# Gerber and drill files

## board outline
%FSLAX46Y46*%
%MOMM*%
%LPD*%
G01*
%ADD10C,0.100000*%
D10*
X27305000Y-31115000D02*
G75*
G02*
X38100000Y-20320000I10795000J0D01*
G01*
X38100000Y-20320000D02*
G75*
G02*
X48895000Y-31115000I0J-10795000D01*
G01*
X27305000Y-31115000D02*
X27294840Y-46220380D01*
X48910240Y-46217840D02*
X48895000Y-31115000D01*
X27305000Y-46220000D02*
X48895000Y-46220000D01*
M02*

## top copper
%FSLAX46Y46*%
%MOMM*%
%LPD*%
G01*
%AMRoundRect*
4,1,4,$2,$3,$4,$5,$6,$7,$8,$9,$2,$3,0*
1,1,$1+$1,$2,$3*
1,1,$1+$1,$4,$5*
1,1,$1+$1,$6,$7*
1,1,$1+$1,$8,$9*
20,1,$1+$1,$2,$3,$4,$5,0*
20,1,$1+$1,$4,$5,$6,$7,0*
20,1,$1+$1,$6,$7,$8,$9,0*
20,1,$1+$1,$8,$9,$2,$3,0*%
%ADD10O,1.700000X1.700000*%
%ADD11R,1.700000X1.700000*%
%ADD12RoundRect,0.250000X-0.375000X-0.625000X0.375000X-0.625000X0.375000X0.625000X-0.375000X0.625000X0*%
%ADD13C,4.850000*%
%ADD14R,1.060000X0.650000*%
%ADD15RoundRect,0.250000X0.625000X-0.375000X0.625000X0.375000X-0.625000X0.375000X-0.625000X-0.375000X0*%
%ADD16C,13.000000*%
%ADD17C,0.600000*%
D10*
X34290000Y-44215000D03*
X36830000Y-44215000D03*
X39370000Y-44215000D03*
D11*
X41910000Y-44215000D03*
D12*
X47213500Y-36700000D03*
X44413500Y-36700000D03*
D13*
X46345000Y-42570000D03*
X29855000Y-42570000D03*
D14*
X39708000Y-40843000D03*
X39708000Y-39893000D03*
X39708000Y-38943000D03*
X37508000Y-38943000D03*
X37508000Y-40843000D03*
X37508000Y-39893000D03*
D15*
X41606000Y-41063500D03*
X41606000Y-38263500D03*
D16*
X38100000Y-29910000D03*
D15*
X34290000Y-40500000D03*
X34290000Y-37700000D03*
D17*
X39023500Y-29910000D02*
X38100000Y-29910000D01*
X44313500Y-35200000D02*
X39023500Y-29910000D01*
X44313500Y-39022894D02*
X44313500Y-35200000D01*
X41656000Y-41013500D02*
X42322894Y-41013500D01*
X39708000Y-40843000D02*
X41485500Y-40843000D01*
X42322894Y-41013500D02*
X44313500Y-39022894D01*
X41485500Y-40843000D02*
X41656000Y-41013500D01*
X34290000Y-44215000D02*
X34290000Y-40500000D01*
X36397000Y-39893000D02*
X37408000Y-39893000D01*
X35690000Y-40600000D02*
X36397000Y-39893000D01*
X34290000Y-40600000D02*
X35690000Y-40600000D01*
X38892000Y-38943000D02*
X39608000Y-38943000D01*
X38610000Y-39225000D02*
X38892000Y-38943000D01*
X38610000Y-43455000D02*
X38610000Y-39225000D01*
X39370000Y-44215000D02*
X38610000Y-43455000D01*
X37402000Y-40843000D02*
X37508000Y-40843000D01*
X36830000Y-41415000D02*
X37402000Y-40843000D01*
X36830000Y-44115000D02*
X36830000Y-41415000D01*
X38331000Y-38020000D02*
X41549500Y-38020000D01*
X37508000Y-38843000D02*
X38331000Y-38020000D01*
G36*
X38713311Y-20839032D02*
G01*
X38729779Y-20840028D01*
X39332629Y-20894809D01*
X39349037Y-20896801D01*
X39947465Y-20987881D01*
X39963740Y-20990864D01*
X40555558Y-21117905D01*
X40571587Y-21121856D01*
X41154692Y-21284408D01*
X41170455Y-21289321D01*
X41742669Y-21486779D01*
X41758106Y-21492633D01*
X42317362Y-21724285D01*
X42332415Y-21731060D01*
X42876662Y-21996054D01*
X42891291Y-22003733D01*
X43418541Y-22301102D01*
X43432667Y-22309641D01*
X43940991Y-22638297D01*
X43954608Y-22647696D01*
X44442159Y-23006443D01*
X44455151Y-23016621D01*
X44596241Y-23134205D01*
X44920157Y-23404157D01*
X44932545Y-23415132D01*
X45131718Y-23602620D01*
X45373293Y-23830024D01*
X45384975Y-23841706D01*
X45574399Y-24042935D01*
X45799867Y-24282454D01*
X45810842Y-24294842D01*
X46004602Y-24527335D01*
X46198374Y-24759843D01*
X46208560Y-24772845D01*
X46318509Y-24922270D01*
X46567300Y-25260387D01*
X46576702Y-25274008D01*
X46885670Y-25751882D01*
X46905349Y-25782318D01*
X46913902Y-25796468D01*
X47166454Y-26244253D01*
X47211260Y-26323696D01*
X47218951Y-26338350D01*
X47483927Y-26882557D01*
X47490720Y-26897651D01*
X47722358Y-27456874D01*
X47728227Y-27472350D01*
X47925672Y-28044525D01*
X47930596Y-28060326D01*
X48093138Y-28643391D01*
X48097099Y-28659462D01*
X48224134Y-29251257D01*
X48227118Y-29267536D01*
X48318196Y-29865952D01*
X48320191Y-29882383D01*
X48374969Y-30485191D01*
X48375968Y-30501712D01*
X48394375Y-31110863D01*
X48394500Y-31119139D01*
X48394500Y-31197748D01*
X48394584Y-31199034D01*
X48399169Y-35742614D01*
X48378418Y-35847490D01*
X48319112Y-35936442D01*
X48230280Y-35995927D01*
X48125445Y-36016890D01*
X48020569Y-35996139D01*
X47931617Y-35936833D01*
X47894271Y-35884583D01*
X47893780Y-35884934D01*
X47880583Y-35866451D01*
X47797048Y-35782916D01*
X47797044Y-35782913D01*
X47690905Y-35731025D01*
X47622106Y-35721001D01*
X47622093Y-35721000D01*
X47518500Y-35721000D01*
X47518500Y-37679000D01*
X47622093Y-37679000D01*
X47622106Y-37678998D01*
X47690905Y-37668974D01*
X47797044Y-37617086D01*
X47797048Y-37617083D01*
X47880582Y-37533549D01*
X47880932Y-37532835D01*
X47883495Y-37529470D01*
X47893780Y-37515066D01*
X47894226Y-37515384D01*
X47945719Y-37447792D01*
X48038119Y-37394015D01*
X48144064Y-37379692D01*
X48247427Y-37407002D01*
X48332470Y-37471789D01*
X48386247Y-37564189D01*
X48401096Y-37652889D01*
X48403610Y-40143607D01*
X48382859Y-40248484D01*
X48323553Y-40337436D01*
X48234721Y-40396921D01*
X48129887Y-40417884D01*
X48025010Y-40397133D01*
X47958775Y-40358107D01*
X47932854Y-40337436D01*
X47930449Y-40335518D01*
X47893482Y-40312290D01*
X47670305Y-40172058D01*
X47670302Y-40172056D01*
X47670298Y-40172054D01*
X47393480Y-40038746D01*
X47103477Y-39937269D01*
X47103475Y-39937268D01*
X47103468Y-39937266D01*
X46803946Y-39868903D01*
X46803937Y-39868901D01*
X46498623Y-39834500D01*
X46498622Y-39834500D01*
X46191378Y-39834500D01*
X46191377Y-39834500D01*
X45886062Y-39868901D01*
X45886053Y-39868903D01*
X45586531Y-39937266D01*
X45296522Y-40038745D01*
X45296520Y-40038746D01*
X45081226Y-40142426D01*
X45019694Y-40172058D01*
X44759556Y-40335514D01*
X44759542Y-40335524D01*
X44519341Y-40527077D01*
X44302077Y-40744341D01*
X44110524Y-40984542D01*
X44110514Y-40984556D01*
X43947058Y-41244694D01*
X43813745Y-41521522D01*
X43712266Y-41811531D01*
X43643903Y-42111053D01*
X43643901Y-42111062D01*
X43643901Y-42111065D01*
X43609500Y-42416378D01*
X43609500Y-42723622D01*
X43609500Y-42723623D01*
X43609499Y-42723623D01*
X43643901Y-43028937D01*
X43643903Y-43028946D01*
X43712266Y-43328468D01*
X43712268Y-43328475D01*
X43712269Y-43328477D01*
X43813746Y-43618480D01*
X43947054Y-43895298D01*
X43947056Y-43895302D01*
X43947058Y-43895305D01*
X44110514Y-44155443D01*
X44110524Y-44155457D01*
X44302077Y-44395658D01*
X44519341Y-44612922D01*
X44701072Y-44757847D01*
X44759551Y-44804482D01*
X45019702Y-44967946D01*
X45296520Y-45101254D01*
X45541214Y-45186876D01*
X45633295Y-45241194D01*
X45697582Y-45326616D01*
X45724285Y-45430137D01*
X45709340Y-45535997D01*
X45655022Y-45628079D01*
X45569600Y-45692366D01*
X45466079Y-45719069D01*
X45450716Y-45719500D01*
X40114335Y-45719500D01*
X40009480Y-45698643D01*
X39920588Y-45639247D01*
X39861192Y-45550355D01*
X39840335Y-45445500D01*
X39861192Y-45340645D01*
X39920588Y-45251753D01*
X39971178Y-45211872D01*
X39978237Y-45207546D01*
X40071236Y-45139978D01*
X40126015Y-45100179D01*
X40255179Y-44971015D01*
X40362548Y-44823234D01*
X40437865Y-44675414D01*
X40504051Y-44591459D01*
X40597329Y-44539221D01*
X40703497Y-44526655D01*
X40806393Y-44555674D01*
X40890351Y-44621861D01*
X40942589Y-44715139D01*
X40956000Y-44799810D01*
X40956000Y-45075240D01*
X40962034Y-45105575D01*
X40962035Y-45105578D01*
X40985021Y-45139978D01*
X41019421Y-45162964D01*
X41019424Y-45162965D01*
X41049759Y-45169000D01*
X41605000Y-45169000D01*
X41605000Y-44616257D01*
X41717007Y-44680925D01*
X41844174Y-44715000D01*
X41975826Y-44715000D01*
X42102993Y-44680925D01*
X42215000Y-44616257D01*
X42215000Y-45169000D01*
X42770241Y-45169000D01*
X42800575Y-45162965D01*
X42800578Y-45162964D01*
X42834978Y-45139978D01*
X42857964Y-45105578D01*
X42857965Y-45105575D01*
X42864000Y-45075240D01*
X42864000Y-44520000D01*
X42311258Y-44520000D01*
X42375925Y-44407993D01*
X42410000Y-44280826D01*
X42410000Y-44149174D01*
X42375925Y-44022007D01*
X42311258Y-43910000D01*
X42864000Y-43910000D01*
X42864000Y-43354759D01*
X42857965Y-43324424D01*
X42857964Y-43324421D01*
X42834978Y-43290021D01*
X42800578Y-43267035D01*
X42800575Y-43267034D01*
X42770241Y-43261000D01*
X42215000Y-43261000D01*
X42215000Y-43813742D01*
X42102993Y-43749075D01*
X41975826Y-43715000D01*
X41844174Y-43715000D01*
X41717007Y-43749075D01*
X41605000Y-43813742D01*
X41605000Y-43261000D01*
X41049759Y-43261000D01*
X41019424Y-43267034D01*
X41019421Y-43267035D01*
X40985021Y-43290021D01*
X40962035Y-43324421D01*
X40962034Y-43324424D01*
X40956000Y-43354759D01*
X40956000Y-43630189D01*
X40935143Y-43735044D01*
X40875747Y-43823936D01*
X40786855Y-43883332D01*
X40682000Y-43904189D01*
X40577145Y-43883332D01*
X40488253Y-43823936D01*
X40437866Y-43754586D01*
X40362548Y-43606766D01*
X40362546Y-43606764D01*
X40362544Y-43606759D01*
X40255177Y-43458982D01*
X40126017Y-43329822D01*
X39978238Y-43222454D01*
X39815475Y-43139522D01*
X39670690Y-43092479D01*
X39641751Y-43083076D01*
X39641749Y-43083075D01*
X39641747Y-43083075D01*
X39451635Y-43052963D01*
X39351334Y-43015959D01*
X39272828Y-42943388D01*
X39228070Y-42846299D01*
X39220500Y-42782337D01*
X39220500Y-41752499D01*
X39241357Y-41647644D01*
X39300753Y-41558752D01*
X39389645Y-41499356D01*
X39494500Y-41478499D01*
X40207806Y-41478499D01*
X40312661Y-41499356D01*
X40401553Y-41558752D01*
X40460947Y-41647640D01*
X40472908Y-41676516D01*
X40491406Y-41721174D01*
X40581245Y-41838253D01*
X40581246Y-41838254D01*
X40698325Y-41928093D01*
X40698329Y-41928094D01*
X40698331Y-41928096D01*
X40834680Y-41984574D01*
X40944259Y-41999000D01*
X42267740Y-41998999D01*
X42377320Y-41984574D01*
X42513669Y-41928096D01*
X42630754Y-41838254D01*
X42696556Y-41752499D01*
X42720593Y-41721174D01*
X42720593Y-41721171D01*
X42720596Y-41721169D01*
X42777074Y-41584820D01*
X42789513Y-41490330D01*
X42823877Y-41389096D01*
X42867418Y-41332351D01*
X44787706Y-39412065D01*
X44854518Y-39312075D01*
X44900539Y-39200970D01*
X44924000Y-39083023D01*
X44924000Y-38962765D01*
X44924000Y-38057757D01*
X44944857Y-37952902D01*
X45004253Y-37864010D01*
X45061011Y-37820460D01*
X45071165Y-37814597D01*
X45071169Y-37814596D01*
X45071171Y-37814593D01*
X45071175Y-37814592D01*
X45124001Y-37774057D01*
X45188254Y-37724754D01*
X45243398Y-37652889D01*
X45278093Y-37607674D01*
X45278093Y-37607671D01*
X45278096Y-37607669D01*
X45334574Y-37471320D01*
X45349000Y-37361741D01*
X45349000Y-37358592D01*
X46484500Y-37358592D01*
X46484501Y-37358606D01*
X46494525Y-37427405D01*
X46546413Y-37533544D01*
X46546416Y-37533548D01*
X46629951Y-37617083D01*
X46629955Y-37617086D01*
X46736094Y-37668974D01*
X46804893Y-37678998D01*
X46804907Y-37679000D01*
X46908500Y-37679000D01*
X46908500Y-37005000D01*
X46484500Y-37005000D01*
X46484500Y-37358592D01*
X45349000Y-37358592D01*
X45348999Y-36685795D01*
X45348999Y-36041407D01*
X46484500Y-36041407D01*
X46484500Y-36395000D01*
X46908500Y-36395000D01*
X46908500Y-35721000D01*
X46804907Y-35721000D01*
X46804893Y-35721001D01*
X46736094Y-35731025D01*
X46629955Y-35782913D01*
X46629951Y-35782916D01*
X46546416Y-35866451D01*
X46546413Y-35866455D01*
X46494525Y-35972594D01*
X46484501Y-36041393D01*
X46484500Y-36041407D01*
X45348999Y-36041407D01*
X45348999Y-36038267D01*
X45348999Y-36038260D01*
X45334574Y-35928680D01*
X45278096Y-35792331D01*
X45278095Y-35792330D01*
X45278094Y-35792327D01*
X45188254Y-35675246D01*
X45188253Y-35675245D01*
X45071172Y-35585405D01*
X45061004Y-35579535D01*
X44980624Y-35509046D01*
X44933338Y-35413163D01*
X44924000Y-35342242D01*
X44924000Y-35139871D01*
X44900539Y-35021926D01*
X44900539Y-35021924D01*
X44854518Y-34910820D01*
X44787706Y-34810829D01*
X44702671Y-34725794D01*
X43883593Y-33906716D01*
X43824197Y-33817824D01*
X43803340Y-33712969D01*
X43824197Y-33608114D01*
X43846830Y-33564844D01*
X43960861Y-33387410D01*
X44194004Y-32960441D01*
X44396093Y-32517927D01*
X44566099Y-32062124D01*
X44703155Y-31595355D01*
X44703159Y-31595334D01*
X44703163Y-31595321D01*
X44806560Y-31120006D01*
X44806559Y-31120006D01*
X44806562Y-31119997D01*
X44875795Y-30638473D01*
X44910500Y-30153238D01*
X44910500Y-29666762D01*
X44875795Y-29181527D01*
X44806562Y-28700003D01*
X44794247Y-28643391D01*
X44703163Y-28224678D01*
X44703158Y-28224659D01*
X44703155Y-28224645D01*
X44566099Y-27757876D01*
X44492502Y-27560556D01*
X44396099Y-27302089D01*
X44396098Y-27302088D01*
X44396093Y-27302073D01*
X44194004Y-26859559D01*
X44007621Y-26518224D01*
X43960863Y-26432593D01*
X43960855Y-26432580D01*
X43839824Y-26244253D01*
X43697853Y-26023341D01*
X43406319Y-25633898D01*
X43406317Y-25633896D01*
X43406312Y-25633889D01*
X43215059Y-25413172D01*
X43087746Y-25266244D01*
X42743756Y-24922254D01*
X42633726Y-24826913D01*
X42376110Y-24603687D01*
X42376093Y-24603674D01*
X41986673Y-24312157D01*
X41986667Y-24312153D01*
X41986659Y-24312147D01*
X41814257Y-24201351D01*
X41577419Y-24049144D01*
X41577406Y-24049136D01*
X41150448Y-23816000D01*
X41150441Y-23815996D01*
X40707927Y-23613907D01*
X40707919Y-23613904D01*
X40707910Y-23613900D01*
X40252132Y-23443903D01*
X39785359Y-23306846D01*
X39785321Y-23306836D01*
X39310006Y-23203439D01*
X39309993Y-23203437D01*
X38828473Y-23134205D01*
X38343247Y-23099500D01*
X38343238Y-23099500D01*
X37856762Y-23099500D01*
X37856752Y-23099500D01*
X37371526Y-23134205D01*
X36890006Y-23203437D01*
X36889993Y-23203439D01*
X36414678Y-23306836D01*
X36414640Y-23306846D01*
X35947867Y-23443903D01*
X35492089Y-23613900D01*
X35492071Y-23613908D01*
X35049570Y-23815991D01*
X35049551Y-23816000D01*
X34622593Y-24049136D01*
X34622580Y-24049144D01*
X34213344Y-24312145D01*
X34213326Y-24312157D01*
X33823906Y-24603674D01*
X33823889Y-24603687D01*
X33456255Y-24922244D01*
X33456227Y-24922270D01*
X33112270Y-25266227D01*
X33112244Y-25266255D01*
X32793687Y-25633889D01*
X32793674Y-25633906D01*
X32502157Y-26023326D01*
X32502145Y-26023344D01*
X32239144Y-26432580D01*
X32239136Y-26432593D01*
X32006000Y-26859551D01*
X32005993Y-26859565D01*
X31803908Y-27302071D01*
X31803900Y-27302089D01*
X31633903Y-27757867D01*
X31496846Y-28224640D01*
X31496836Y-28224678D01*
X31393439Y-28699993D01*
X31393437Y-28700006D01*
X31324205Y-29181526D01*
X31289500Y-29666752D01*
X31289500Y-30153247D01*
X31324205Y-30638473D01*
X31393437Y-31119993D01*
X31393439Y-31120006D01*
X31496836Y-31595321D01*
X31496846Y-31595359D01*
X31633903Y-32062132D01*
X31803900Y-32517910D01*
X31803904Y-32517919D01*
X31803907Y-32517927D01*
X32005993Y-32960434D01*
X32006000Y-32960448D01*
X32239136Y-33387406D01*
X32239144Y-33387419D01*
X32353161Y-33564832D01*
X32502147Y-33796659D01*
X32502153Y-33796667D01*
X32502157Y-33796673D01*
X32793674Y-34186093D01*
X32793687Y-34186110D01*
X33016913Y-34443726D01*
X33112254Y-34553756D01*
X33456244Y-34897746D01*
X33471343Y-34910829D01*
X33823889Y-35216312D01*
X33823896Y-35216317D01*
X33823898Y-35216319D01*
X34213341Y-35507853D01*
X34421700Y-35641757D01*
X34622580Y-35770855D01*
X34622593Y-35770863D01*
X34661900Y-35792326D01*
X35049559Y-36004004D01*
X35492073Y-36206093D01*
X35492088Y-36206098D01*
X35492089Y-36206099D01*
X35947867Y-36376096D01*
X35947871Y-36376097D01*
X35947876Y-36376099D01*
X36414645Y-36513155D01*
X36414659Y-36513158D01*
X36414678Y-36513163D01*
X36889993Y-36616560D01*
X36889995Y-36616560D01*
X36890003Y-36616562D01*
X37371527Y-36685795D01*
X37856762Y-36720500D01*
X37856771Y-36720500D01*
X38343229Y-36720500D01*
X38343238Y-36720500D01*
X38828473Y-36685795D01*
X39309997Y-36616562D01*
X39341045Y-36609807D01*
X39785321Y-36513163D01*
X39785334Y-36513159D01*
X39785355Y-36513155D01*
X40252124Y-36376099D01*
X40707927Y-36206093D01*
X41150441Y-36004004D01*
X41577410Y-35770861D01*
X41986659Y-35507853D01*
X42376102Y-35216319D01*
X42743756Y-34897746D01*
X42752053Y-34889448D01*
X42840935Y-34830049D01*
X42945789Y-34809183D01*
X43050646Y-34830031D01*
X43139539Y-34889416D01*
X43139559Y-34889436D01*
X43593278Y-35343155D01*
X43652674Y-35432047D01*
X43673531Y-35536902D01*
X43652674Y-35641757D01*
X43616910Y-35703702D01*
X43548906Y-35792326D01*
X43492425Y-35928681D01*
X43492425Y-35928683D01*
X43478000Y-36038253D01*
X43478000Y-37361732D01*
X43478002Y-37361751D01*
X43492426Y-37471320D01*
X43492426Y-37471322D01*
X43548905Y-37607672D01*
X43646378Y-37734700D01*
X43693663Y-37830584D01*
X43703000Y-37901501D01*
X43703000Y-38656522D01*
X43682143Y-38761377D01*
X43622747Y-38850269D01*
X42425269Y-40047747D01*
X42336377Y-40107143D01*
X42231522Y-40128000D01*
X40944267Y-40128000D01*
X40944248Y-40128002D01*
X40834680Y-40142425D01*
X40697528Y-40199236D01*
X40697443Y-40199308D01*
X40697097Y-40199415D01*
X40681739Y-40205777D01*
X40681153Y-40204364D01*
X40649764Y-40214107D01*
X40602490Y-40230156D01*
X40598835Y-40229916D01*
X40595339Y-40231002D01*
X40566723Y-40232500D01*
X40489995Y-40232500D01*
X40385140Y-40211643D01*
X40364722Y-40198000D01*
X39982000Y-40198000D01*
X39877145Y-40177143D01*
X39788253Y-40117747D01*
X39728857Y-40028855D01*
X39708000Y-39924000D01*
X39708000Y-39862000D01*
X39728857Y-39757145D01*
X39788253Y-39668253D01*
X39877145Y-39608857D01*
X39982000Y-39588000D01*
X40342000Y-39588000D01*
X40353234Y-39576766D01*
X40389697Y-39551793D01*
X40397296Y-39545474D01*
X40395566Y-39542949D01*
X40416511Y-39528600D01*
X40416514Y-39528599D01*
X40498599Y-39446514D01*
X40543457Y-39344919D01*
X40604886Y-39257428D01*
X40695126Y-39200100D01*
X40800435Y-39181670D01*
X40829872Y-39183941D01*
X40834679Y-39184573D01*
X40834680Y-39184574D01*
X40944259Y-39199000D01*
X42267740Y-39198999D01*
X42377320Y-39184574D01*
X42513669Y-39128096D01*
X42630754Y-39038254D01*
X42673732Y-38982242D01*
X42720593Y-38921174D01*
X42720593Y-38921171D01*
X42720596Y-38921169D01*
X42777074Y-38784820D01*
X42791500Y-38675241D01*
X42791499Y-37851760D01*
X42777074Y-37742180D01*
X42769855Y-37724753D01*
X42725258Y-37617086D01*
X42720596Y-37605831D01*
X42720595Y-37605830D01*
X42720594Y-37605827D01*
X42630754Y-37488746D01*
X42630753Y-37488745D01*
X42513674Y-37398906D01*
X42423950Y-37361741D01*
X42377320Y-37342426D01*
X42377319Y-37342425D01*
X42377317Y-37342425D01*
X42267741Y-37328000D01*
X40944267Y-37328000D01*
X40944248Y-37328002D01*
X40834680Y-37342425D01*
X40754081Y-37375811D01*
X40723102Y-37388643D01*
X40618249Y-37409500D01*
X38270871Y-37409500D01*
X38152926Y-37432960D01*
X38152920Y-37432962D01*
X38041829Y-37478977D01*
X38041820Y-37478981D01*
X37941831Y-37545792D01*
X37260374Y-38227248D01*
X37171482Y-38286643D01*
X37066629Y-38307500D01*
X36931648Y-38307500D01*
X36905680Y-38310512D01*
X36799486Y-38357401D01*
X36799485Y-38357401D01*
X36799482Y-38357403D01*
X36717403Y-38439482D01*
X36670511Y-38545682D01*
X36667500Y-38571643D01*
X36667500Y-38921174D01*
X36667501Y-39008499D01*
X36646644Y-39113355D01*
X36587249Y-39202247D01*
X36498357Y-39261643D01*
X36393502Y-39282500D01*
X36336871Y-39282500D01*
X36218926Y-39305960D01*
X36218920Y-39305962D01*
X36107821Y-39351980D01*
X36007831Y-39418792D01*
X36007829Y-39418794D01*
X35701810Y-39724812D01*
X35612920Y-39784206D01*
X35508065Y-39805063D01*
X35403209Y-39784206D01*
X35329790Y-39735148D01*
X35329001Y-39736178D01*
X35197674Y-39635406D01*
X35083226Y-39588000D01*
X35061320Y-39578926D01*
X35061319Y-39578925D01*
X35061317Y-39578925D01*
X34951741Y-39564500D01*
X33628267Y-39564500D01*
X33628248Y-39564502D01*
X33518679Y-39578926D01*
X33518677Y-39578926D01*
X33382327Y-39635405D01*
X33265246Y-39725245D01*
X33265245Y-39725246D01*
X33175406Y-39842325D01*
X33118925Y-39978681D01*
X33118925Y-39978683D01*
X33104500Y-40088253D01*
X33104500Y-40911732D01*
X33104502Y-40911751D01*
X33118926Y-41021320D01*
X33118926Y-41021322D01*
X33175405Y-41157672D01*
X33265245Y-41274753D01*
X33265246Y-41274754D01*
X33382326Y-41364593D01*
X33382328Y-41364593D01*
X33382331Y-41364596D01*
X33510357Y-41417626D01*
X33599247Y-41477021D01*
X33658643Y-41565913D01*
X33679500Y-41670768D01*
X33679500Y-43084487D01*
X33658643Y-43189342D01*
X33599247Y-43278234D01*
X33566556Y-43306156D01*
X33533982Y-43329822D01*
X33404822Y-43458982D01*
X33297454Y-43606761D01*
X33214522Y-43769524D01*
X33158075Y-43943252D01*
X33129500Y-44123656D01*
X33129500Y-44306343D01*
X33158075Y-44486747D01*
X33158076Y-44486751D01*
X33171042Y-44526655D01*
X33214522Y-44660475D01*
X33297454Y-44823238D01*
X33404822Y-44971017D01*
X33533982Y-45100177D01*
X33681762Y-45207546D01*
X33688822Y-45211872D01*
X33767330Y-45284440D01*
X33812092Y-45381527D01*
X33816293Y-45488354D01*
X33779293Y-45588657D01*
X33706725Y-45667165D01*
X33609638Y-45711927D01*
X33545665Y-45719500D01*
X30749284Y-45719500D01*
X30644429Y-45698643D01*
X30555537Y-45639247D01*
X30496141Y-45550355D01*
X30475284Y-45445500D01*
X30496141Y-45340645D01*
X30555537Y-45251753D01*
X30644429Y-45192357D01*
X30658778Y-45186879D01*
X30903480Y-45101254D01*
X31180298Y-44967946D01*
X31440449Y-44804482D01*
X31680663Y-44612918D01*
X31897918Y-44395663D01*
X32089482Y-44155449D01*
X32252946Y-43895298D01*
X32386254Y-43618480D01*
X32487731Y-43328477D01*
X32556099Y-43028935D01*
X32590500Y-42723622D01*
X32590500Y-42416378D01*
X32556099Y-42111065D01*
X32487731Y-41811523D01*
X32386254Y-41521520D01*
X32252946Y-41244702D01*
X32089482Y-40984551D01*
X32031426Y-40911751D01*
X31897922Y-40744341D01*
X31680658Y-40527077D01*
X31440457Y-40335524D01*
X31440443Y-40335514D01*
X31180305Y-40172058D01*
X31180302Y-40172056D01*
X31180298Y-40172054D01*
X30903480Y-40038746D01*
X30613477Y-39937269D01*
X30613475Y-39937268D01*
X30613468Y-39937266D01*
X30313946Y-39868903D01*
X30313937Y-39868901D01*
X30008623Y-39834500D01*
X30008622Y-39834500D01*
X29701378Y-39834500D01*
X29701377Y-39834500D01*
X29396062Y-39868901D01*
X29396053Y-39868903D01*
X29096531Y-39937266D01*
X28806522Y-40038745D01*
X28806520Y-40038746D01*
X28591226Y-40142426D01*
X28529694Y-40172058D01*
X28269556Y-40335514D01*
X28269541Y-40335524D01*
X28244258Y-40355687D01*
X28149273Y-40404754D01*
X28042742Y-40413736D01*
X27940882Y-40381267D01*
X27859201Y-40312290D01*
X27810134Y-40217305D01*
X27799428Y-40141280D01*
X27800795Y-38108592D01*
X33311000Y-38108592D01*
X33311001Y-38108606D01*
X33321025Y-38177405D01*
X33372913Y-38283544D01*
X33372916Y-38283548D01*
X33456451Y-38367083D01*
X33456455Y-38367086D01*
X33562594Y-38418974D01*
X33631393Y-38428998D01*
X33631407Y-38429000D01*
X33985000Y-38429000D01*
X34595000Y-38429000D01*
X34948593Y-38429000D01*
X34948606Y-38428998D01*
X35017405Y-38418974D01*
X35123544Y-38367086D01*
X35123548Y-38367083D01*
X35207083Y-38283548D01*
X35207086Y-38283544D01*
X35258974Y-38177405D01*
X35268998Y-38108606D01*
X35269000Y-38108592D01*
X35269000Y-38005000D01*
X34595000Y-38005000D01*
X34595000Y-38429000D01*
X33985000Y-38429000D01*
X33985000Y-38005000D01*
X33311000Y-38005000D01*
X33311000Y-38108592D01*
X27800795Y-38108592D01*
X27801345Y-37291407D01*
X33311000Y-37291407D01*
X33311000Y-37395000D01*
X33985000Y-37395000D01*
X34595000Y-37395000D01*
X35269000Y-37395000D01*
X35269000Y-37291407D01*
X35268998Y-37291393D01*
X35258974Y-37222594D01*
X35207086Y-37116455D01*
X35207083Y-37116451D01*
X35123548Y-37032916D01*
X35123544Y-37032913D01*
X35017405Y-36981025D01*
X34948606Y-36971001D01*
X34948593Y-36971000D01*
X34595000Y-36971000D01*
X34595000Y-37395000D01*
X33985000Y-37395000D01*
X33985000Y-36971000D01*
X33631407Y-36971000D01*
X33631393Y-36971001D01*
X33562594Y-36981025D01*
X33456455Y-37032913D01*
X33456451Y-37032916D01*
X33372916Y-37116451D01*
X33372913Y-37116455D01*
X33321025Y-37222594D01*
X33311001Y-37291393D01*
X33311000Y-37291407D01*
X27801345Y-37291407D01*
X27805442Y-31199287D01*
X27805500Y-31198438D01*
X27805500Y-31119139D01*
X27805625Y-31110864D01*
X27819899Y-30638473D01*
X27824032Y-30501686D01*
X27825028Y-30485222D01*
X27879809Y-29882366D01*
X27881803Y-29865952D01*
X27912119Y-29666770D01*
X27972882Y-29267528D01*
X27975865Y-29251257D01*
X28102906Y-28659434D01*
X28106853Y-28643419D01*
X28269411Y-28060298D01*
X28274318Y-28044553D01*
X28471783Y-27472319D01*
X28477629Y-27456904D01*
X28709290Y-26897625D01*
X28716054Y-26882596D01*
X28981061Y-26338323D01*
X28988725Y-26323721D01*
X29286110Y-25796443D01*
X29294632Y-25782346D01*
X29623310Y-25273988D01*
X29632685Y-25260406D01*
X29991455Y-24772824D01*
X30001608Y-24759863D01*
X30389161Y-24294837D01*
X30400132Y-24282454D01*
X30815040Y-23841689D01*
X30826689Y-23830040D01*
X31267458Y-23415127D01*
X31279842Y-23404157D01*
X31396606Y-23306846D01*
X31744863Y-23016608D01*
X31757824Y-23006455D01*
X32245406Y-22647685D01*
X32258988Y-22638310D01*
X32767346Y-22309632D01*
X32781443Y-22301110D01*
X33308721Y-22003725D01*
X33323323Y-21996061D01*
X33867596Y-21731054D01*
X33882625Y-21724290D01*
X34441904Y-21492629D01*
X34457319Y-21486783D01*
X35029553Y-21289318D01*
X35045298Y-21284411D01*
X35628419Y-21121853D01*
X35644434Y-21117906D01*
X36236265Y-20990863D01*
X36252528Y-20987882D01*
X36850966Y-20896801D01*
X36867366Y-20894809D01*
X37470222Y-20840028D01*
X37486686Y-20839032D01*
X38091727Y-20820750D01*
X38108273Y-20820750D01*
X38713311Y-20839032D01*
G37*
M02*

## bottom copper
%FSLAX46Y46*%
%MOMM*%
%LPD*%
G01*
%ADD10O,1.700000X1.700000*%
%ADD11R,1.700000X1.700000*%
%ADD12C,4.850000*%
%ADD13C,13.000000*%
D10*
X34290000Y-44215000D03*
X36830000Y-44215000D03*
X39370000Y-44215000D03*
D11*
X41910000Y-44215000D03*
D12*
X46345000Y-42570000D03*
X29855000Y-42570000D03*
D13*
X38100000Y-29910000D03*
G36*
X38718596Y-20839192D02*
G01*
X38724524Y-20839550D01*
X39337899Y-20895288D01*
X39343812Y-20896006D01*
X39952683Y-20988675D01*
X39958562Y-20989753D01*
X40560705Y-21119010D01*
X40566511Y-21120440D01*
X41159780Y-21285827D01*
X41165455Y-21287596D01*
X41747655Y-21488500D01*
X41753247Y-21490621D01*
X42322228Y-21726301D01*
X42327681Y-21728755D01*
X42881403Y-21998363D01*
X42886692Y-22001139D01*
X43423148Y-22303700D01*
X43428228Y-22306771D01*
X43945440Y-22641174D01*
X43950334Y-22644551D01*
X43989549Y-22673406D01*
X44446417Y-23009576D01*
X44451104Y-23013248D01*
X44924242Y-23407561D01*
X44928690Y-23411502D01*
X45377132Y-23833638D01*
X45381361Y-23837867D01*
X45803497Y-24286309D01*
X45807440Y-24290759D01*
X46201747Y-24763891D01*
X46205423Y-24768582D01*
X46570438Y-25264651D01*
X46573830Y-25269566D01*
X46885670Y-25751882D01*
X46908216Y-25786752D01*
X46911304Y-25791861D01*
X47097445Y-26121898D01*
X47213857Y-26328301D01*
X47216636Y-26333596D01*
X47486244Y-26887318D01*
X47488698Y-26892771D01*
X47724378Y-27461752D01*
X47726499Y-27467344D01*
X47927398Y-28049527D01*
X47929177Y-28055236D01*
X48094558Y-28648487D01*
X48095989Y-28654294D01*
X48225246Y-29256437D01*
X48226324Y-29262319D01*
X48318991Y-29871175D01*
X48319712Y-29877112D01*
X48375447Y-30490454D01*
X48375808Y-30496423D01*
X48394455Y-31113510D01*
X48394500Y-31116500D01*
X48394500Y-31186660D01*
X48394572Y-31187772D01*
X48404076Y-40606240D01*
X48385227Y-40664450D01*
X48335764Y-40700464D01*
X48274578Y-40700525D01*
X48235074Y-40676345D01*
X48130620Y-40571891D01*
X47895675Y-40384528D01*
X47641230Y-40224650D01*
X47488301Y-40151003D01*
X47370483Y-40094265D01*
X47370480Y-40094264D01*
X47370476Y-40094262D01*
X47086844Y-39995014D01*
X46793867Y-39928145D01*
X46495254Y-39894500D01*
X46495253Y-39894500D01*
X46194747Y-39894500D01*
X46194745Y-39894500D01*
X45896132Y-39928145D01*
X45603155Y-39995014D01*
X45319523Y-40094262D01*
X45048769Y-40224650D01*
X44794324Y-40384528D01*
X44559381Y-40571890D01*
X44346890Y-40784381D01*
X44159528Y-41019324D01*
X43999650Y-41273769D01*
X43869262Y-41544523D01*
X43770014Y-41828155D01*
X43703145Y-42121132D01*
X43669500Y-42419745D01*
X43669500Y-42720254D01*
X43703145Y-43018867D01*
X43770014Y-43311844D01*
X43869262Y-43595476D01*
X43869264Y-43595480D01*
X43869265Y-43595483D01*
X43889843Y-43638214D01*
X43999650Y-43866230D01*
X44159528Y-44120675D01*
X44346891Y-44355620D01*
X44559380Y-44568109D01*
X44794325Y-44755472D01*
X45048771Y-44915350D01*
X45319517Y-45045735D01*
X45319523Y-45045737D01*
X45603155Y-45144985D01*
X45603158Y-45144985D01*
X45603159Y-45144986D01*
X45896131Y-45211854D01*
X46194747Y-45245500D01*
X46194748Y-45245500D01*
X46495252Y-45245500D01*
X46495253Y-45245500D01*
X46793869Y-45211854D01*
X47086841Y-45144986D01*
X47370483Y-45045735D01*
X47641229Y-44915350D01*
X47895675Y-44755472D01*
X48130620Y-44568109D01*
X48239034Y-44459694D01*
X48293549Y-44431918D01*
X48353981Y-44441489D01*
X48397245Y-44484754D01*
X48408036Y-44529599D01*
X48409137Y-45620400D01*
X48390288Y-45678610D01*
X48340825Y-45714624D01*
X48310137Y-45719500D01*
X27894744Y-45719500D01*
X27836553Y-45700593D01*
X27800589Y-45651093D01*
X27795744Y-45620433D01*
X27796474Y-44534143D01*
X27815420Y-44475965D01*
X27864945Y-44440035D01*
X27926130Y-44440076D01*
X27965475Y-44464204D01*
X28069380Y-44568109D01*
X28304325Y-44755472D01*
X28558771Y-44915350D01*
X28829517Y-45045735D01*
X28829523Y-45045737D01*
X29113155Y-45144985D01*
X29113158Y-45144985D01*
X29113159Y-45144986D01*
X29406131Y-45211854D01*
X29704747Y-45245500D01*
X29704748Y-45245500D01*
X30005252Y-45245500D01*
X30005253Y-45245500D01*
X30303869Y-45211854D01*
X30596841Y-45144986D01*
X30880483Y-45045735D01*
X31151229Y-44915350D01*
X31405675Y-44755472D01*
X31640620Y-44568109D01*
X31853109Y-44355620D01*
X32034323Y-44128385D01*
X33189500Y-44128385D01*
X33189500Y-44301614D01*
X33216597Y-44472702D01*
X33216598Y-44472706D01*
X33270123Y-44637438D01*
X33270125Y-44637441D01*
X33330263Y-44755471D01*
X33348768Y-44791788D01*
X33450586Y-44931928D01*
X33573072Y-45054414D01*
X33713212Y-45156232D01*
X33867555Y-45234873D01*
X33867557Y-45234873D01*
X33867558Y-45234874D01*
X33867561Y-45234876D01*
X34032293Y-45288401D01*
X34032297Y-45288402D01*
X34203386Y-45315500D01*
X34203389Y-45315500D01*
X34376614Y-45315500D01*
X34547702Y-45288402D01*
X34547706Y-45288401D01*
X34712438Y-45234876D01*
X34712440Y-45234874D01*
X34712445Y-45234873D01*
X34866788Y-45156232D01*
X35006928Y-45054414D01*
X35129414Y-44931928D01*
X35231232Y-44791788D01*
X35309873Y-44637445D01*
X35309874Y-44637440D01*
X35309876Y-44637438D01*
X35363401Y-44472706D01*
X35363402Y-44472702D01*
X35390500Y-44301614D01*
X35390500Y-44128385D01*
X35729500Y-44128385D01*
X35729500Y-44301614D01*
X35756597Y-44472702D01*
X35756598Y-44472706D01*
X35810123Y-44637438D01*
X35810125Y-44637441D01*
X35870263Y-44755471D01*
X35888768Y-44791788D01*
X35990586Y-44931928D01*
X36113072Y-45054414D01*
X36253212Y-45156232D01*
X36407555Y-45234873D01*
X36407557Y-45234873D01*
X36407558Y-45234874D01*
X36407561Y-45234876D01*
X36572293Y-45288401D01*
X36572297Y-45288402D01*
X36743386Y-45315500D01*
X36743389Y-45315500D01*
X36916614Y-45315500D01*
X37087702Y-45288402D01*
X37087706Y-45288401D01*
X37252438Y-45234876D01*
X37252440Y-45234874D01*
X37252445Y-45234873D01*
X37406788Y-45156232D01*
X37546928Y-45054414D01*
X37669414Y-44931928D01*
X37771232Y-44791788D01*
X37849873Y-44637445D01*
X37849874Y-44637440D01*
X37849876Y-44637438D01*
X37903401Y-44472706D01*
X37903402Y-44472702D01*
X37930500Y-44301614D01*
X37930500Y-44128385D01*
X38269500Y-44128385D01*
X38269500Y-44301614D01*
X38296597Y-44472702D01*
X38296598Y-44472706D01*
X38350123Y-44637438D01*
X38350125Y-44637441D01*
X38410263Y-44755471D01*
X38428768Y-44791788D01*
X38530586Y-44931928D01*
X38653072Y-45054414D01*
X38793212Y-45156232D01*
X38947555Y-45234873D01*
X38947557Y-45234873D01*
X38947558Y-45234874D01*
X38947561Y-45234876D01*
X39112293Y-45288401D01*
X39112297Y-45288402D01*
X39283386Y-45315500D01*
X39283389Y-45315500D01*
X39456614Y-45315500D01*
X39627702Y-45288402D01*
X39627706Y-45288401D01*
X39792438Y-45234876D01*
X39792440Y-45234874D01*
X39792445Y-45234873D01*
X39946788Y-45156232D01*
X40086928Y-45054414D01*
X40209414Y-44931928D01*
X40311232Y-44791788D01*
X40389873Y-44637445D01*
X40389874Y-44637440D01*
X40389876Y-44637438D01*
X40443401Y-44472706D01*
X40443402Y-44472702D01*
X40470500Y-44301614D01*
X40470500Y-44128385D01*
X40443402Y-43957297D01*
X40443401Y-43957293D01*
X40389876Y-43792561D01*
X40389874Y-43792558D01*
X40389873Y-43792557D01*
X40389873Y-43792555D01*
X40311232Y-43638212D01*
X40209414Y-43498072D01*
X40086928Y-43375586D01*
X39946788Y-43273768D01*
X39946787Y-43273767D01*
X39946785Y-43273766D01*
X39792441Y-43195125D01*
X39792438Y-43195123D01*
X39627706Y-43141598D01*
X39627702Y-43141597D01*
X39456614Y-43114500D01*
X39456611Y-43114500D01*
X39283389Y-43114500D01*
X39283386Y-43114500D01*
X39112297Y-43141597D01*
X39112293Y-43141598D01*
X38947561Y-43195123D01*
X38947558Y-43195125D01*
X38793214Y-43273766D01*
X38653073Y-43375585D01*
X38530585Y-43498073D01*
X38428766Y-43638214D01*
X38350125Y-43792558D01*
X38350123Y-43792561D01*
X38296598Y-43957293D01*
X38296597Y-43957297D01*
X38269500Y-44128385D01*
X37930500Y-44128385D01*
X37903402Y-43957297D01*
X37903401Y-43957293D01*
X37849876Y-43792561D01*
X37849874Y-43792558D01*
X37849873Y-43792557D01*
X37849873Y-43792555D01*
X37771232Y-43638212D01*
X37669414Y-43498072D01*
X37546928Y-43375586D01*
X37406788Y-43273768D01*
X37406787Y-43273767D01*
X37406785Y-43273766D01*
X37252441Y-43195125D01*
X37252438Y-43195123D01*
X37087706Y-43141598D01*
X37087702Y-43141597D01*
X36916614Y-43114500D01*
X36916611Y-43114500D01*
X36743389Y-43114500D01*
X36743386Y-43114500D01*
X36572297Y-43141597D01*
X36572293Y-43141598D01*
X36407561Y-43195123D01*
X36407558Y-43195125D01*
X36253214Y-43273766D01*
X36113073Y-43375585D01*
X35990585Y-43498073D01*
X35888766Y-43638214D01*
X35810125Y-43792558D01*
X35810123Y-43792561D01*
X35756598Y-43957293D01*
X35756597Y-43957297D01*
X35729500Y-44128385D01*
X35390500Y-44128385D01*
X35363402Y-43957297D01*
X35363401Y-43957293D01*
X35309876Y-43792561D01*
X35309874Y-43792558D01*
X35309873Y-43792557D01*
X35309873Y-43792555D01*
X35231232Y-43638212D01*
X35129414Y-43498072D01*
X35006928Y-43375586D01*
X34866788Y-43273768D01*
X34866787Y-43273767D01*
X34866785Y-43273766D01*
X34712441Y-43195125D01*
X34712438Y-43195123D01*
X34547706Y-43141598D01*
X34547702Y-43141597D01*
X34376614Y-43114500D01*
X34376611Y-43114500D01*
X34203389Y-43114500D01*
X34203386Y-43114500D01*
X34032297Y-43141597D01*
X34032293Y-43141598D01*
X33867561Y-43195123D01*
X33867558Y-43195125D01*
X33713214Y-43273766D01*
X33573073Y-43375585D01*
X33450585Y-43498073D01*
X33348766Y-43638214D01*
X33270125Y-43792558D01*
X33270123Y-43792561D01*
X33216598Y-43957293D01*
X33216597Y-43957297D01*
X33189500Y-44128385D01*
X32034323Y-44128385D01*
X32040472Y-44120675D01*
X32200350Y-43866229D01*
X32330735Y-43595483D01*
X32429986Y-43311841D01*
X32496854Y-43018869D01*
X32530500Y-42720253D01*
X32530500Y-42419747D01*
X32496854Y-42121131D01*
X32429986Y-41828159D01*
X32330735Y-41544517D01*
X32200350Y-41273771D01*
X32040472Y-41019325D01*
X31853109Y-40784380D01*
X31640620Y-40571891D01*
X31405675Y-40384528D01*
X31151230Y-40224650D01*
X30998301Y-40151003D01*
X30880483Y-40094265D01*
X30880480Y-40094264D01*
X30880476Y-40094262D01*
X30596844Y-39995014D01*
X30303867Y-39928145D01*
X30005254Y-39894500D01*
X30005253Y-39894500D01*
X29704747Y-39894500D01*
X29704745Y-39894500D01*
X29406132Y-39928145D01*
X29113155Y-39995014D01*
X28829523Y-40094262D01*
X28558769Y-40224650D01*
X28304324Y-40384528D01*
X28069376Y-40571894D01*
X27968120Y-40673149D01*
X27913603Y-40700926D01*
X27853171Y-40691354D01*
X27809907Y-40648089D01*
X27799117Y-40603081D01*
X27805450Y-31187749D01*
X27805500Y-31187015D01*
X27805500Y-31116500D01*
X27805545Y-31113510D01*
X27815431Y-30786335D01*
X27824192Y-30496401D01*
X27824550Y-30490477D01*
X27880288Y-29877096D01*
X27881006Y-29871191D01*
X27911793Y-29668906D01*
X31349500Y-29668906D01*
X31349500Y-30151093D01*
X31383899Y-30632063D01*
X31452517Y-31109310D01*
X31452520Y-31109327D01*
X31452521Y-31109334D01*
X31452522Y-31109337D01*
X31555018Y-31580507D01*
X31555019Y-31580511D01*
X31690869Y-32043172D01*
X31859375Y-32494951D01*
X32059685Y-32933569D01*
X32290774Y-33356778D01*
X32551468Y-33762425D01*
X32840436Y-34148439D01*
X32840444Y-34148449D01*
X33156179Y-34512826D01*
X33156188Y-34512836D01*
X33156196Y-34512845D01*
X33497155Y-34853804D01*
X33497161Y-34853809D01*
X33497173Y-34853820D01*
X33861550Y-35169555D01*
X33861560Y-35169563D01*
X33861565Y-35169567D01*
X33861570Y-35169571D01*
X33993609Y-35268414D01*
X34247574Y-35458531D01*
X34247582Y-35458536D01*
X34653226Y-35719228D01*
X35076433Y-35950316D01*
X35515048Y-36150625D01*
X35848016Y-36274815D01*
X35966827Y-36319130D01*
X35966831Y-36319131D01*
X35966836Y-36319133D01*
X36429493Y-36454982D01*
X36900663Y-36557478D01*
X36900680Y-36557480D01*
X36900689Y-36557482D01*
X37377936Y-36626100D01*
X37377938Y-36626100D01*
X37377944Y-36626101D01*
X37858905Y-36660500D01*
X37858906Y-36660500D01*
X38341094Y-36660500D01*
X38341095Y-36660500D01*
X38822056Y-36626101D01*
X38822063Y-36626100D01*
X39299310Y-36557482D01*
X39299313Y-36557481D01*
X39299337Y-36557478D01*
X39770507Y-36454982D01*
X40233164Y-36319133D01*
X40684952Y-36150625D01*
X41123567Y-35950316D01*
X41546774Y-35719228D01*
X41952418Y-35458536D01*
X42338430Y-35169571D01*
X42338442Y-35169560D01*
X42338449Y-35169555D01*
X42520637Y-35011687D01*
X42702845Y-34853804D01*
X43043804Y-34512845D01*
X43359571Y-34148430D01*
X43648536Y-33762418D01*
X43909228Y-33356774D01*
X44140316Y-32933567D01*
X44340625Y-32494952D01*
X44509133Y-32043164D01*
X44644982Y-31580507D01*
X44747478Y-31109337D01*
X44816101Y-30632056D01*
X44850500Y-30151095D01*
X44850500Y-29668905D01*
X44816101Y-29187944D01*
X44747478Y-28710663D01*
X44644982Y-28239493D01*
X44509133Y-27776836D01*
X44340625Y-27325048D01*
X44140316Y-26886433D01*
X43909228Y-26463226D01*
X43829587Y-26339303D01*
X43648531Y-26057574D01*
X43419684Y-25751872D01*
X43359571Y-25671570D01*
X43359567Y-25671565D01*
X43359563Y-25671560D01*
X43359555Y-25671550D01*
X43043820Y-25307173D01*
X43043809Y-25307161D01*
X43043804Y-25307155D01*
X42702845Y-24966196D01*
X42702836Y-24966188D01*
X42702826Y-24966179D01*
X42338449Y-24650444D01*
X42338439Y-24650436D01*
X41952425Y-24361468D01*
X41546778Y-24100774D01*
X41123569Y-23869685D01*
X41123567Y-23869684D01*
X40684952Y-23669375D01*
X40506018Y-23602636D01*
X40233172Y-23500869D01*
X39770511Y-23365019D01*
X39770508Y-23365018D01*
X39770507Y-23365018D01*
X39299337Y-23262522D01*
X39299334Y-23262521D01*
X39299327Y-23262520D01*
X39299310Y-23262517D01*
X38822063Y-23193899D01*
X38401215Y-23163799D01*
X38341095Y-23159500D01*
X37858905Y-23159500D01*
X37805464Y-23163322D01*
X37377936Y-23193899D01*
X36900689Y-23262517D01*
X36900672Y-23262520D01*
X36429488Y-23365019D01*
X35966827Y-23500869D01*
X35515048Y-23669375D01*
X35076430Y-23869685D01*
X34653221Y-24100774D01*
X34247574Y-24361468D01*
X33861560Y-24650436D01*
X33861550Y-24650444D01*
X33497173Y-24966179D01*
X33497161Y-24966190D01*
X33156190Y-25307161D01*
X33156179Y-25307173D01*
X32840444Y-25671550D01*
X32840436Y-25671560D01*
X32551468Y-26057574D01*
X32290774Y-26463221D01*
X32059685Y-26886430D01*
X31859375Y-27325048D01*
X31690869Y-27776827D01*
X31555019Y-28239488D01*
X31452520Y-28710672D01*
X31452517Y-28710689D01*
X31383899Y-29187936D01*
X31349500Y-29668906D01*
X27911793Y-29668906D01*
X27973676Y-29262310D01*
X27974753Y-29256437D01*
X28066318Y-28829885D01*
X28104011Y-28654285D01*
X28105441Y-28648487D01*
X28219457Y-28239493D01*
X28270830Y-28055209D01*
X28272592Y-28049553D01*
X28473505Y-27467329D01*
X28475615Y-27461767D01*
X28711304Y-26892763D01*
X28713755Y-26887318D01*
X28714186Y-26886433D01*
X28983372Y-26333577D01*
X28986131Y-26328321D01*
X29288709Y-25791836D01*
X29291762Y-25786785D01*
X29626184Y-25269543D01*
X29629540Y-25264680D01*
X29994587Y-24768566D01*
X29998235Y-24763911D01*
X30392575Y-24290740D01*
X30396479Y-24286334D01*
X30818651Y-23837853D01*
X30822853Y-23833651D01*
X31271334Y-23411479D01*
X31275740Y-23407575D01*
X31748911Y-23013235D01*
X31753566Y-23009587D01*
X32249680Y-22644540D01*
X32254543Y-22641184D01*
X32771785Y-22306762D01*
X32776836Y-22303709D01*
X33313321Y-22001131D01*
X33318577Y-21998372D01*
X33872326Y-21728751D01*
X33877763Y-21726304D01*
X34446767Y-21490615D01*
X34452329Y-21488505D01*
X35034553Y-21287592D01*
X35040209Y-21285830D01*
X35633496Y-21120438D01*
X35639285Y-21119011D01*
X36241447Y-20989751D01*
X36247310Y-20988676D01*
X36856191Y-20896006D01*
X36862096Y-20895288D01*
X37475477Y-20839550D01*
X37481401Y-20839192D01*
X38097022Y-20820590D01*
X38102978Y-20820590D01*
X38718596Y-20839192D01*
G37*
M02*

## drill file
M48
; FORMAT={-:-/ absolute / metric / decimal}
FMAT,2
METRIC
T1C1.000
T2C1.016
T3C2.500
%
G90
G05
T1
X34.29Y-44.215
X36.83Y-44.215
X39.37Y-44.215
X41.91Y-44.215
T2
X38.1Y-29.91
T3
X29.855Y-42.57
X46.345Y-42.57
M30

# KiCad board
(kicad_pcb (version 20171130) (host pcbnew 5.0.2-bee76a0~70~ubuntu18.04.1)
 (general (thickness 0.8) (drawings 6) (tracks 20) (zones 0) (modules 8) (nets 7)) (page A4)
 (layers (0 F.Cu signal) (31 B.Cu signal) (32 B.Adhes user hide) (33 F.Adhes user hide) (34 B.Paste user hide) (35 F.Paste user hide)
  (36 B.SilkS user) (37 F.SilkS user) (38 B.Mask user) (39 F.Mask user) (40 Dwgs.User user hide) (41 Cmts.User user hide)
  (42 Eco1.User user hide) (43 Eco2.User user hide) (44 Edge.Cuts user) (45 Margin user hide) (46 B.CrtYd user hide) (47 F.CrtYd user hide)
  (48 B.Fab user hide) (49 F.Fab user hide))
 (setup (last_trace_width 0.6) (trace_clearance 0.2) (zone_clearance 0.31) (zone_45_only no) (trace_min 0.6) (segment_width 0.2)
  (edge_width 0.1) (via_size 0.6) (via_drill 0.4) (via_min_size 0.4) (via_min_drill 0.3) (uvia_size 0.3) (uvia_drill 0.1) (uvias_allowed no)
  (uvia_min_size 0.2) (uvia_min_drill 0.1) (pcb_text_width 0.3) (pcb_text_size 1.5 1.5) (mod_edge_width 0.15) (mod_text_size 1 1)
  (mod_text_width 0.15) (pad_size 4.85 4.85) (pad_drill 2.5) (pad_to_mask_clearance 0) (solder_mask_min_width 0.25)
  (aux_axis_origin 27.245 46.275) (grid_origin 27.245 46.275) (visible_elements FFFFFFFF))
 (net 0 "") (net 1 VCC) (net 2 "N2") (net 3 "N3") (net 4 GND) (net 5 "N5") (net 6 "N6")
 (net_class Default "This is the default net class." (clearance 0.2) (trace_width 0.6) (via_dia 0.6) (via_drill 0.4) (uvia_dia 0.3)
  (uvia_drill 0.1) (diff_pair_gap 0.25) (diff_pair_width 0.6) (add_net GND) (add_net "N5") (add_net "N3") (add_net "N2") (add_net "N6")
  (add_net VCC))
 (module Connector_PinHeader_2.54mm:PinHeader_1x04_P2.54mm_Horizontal (layer F.Cu) (at 41.91 44.215 270)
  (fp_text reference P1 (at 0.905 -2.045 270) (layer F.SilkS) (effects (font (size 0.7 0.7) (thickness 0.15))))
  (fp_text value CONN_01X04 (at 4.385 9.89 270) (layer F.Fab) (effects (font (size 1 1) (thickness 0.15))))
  (pad 4 thru_hole oval (at 0 7.62 270) (size 1.7 1.7) (drill 1) (layers *.Cu *.Mask) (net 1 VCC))
  (pad 3 thru_hole oval (at 0 5.08 270) (size 1.7 1.7) (drill 1) (layers *.Cu *.Mask) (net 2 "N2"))
  (pad 2 thru_hole oval (at 0 2.54 270) (size 1.7 1.7) (drill 1) (layers *.Cu *.Mask) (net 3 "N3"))
  (pad 1 thru_hole rect (at 0 0 270) (size 1.7 1.7) (drill 1) (layers *.Cu *.Mask) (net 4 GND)))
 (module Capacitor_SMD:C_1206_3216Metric (layer F.Cu) (at 45.8135 36.7)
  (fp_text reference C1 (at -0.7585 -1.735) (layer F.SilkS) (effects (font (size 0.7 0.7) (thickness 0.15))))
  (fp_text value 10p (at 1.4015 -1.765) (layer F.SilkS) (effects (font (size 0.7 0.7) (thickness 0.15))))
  (pad 2 smd roundrect (at 1.4 0) (size 1.25 1.75) (layers F.Cu F.Paste F.Mask) (roundrect_rratio 0.2) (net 4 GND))
  (pad 1 smd roundrect (at -1.4 0) (size 1.25 1.75) (layers F.Cu F.Paste F.Mask) (roundrect_rratio 0.2) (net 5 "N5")))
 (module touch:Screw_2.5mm (layer F.Cu) (at 46.345 42.58 90)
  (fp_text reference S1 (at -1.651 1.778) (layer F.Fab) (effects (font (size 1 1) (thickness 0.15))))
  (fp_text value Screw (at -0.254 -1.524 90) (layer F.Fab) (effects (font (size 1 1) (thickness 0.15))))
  (pad 1 thru_hole circle (at 0.01 0 90) (size 4.85 4.85) (drill 2.5) (layers *.Cu *.Mask F.SilkS)))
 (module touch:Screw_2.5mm (layer F.Cu) (at 29.855 42.57 90)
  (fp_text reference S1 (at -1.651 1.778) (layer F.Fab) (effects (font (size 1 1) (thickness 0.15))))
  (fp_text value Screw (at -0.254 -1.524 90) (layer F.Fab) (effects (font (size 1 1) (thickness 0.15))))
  (pad 1 thru_hole circle (at 0 0 90) (size 4.85 4.85) (drill 2.5) (layers *.Cu *.Mask F.SilkS)))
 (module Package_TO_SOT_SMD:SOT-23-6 (layer F.Cu) (at 38.608 39.893 180)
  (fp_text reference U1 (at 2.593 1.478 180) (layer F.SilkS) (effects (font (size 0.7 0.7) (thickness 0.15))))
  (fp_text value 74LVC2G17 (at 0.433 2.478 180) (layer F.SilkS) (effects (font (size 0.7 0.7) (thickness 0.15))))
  (pad 1 smd rect (at -1.1 -0.95 180) (size 1.06 0.65) (layers F.Cu F.Paste F.Mask) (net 5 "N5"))
  (pad 2 smd rect (at -1.1 0 180) (size 1.06 0.65) (layers F.Cu F.Paste F.Mask) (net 4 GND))
  (pad 3 smd rect (at -1.1 0.95 180) (size 1.06 0.65) (layers F.Cu F.Paste F.Mask) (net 3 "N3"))
  (pad 4 smd rect (at 1.1 0.95 180) (size 1.06 0.65) (layers F.Cu F.Paste F.Mask) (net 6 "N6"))
  (pad 6 smd rect (at 1.1 -0.95 180) (size 1.06 0.65) (layers F.Cu F.Paste F.Mask) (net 2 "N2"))
  (pad 5 smd rect (at 1.1 0 180) (size 1.06 0.65) (layers F.Cu F.Paste F.Mask) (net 1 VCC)))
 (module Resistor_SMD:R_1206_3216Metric (layer F.Cu) (at 41.606 39.6635 90)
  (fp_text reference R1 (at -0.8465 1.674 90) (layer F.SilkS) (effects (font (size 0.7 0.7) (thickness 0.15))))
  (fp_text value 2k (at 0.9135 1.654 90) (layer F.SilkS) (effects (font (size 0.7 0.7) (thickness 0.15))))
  (pad 1 smd roundrect (at -1.4 0 90) (size 1.25 1.75) (layers F.Cu F.Paste F.Mask) (roundrect_rratio 0.2) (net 5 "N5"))
  (pad 2 smd roundrect (at 1.4 0 90) (size 1.25 1.75) (layers F.Cu F.Paste F.Mask) (roundrect_rratio 0.2) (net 6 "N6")))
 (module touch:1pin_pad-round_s (layer F.Cu) (at 38.1 29.91 90)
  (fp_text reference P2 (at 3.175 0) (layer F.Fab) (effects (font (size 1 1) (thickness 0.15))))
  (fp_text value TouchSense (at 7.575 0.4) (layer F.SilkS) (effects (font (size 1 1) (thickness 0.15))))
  (pad 1 thru_hole circle (at 0 0 90) (size 13 13) (drill 1.016) (layers *.Cu *.Mask F.SilkS) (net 5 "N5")))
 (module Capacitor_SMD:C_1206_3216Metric (layer F.Cu) (at 34.29 39.1 90)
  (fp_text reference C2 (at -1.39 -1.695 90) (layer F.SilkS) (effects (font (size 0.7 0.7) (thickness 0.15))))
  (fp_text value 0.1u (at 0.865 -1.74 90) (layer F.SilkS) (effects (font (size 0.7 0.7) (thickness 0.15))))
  (pad 1 smd roundrect (at -1.4 0 90) (size 1.25 1.75) (layers F.Cu F.Paste F.Mask) (roundrect_rratio 0.2) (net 1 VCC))
  (pad 2 smd roundrect (at 1.4 0 90) (size 1.25 1.75) (layers F.Cu F.Paste F.Mask) (roundrect_rratio 0.2) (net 4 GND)))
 (gr_arc (start 38.1 31.115) (end 27.305 31.115) (angle 90) (layer Edge.Cuts) (width 0.1))
 (gr_arc (start 38.1 31.115) (end 38.1 20.32) (angle 90) (layer Edge.Cuts) (width 0.1))
 (gr_line (start 27.305 31.115) (end 27.29484 46.22038) (angle 90) (layer Edge.Cuts) (width 0.1))
 (gr_line (start 48.91024 46.21784) (end 48.895 31.115) (angle 90) (layer Edge.Cuts) (width 0.1))
 (gr_line (start 27.305 46.22) (end 48.895 46.22) (angle 90) (layer Edge.Cuts) (width 0.1))
 (segment (start 39.0235 29.91) (end 38.1 29.91) (width 0.6) (layer F.Cu) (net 5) (status 30))
 (segment (start 44.3135 35.2) (end 39.0235 29.91) (width 0.6) (layer F.Cu) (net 5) (status 20))
 (segment (start 44.3135 39.022894) (end 44.3135 35.2) (width 0.6) (layer F.Cu) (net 5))
 (segment (start 41.656 41.0135) (end 42.322894 41.0135) (width 0.6) (layer F.Cu) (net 5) (status 30))
 (segment (start 39.708 40.843) (end 41.4855 40.843) (width 0.6) (layer F.Cu) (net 5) (status 30))
 (segment (start 42.322894 41.0135) (end 44.3135 39.022894) (width 0.6) (layer F.Cu) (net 5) (status 10))
 (segment (start 41.4855 40.843) (end 41.656 41.0135) (width 0.6) (layer F.Cu) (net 5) (status 30))
 (segment (start 34.29 44.215) (end 34.29 40.5) (width 0.6) (layer F.Cu) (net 1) (status 30))
 (segment (start 36.397 39.893) (end 37.408 39.893) (width 0.6) (layer F.Cu) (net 1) (status 20))
 (segment (start 35.69 40.6) (end 36.397 39.893) (width 0.6) (layer F.Cu) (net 1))
 (segment (start 34.29 40.6) (end 35.69 40.6) (width 0.6) (layer F.Cu) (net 1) (status 10))
 (segment (start 38.892 38.943) (end 39.608 38.943) (width 0.6) (layer F.Cu) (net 3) (status 20))
 (segment (start 38.61 39.225) (end 38.892 38.943) (width 0.6) (layer F.Cu) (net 3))
 (segment (start 38.61 43.455) (end 38.61 39.225) (width 0.6) (layer F.Cu) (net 3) (status 10))
 (segment (start 39.37 44.215) (end 38.61 43.455) (width 0.6) (layer F.Cu) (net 3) (status 30))
 (segment (start 37.402 40.843) (end 37.508 40.843) (width 0.6) (layer F.Cu) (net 2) (status 30))
 (segment (start 36.83 41.415) (end 37.402 40.843) (width 0.6) (layer F.Cu) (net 2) (status 20))
 (segment (start 36.83 44.115) (end 36.83 41.415) (width 0.6) (layer F.Cu) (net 2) (status 10))
 (segment (start 38.331 38.02) (end 41.5495 38.02) (width 0.6) (layer F.Cu) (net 6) (status 20))
 (segment (start 37.508 38.843) (end 38.331 38.02) (width 0.6) (layer F.Cu) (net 6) (status 10))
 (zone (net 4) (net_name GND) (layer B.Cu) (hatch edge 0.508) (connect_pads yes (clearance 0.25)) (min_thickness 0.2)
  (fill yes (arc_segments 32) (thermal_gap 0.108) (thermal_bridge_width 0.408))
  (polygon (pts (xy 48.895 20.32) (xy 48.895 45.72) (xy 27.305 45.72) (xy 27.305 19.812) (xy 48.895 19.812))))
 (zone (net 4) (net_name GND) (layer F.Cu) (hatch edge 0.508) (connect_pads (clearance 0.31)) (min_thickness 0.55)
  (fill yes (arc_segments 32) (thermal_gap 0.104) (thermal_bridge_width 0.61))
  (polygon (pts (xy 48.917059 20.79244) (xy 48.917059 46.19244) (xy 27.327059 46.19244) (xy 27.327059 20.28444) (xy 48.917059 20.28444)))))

